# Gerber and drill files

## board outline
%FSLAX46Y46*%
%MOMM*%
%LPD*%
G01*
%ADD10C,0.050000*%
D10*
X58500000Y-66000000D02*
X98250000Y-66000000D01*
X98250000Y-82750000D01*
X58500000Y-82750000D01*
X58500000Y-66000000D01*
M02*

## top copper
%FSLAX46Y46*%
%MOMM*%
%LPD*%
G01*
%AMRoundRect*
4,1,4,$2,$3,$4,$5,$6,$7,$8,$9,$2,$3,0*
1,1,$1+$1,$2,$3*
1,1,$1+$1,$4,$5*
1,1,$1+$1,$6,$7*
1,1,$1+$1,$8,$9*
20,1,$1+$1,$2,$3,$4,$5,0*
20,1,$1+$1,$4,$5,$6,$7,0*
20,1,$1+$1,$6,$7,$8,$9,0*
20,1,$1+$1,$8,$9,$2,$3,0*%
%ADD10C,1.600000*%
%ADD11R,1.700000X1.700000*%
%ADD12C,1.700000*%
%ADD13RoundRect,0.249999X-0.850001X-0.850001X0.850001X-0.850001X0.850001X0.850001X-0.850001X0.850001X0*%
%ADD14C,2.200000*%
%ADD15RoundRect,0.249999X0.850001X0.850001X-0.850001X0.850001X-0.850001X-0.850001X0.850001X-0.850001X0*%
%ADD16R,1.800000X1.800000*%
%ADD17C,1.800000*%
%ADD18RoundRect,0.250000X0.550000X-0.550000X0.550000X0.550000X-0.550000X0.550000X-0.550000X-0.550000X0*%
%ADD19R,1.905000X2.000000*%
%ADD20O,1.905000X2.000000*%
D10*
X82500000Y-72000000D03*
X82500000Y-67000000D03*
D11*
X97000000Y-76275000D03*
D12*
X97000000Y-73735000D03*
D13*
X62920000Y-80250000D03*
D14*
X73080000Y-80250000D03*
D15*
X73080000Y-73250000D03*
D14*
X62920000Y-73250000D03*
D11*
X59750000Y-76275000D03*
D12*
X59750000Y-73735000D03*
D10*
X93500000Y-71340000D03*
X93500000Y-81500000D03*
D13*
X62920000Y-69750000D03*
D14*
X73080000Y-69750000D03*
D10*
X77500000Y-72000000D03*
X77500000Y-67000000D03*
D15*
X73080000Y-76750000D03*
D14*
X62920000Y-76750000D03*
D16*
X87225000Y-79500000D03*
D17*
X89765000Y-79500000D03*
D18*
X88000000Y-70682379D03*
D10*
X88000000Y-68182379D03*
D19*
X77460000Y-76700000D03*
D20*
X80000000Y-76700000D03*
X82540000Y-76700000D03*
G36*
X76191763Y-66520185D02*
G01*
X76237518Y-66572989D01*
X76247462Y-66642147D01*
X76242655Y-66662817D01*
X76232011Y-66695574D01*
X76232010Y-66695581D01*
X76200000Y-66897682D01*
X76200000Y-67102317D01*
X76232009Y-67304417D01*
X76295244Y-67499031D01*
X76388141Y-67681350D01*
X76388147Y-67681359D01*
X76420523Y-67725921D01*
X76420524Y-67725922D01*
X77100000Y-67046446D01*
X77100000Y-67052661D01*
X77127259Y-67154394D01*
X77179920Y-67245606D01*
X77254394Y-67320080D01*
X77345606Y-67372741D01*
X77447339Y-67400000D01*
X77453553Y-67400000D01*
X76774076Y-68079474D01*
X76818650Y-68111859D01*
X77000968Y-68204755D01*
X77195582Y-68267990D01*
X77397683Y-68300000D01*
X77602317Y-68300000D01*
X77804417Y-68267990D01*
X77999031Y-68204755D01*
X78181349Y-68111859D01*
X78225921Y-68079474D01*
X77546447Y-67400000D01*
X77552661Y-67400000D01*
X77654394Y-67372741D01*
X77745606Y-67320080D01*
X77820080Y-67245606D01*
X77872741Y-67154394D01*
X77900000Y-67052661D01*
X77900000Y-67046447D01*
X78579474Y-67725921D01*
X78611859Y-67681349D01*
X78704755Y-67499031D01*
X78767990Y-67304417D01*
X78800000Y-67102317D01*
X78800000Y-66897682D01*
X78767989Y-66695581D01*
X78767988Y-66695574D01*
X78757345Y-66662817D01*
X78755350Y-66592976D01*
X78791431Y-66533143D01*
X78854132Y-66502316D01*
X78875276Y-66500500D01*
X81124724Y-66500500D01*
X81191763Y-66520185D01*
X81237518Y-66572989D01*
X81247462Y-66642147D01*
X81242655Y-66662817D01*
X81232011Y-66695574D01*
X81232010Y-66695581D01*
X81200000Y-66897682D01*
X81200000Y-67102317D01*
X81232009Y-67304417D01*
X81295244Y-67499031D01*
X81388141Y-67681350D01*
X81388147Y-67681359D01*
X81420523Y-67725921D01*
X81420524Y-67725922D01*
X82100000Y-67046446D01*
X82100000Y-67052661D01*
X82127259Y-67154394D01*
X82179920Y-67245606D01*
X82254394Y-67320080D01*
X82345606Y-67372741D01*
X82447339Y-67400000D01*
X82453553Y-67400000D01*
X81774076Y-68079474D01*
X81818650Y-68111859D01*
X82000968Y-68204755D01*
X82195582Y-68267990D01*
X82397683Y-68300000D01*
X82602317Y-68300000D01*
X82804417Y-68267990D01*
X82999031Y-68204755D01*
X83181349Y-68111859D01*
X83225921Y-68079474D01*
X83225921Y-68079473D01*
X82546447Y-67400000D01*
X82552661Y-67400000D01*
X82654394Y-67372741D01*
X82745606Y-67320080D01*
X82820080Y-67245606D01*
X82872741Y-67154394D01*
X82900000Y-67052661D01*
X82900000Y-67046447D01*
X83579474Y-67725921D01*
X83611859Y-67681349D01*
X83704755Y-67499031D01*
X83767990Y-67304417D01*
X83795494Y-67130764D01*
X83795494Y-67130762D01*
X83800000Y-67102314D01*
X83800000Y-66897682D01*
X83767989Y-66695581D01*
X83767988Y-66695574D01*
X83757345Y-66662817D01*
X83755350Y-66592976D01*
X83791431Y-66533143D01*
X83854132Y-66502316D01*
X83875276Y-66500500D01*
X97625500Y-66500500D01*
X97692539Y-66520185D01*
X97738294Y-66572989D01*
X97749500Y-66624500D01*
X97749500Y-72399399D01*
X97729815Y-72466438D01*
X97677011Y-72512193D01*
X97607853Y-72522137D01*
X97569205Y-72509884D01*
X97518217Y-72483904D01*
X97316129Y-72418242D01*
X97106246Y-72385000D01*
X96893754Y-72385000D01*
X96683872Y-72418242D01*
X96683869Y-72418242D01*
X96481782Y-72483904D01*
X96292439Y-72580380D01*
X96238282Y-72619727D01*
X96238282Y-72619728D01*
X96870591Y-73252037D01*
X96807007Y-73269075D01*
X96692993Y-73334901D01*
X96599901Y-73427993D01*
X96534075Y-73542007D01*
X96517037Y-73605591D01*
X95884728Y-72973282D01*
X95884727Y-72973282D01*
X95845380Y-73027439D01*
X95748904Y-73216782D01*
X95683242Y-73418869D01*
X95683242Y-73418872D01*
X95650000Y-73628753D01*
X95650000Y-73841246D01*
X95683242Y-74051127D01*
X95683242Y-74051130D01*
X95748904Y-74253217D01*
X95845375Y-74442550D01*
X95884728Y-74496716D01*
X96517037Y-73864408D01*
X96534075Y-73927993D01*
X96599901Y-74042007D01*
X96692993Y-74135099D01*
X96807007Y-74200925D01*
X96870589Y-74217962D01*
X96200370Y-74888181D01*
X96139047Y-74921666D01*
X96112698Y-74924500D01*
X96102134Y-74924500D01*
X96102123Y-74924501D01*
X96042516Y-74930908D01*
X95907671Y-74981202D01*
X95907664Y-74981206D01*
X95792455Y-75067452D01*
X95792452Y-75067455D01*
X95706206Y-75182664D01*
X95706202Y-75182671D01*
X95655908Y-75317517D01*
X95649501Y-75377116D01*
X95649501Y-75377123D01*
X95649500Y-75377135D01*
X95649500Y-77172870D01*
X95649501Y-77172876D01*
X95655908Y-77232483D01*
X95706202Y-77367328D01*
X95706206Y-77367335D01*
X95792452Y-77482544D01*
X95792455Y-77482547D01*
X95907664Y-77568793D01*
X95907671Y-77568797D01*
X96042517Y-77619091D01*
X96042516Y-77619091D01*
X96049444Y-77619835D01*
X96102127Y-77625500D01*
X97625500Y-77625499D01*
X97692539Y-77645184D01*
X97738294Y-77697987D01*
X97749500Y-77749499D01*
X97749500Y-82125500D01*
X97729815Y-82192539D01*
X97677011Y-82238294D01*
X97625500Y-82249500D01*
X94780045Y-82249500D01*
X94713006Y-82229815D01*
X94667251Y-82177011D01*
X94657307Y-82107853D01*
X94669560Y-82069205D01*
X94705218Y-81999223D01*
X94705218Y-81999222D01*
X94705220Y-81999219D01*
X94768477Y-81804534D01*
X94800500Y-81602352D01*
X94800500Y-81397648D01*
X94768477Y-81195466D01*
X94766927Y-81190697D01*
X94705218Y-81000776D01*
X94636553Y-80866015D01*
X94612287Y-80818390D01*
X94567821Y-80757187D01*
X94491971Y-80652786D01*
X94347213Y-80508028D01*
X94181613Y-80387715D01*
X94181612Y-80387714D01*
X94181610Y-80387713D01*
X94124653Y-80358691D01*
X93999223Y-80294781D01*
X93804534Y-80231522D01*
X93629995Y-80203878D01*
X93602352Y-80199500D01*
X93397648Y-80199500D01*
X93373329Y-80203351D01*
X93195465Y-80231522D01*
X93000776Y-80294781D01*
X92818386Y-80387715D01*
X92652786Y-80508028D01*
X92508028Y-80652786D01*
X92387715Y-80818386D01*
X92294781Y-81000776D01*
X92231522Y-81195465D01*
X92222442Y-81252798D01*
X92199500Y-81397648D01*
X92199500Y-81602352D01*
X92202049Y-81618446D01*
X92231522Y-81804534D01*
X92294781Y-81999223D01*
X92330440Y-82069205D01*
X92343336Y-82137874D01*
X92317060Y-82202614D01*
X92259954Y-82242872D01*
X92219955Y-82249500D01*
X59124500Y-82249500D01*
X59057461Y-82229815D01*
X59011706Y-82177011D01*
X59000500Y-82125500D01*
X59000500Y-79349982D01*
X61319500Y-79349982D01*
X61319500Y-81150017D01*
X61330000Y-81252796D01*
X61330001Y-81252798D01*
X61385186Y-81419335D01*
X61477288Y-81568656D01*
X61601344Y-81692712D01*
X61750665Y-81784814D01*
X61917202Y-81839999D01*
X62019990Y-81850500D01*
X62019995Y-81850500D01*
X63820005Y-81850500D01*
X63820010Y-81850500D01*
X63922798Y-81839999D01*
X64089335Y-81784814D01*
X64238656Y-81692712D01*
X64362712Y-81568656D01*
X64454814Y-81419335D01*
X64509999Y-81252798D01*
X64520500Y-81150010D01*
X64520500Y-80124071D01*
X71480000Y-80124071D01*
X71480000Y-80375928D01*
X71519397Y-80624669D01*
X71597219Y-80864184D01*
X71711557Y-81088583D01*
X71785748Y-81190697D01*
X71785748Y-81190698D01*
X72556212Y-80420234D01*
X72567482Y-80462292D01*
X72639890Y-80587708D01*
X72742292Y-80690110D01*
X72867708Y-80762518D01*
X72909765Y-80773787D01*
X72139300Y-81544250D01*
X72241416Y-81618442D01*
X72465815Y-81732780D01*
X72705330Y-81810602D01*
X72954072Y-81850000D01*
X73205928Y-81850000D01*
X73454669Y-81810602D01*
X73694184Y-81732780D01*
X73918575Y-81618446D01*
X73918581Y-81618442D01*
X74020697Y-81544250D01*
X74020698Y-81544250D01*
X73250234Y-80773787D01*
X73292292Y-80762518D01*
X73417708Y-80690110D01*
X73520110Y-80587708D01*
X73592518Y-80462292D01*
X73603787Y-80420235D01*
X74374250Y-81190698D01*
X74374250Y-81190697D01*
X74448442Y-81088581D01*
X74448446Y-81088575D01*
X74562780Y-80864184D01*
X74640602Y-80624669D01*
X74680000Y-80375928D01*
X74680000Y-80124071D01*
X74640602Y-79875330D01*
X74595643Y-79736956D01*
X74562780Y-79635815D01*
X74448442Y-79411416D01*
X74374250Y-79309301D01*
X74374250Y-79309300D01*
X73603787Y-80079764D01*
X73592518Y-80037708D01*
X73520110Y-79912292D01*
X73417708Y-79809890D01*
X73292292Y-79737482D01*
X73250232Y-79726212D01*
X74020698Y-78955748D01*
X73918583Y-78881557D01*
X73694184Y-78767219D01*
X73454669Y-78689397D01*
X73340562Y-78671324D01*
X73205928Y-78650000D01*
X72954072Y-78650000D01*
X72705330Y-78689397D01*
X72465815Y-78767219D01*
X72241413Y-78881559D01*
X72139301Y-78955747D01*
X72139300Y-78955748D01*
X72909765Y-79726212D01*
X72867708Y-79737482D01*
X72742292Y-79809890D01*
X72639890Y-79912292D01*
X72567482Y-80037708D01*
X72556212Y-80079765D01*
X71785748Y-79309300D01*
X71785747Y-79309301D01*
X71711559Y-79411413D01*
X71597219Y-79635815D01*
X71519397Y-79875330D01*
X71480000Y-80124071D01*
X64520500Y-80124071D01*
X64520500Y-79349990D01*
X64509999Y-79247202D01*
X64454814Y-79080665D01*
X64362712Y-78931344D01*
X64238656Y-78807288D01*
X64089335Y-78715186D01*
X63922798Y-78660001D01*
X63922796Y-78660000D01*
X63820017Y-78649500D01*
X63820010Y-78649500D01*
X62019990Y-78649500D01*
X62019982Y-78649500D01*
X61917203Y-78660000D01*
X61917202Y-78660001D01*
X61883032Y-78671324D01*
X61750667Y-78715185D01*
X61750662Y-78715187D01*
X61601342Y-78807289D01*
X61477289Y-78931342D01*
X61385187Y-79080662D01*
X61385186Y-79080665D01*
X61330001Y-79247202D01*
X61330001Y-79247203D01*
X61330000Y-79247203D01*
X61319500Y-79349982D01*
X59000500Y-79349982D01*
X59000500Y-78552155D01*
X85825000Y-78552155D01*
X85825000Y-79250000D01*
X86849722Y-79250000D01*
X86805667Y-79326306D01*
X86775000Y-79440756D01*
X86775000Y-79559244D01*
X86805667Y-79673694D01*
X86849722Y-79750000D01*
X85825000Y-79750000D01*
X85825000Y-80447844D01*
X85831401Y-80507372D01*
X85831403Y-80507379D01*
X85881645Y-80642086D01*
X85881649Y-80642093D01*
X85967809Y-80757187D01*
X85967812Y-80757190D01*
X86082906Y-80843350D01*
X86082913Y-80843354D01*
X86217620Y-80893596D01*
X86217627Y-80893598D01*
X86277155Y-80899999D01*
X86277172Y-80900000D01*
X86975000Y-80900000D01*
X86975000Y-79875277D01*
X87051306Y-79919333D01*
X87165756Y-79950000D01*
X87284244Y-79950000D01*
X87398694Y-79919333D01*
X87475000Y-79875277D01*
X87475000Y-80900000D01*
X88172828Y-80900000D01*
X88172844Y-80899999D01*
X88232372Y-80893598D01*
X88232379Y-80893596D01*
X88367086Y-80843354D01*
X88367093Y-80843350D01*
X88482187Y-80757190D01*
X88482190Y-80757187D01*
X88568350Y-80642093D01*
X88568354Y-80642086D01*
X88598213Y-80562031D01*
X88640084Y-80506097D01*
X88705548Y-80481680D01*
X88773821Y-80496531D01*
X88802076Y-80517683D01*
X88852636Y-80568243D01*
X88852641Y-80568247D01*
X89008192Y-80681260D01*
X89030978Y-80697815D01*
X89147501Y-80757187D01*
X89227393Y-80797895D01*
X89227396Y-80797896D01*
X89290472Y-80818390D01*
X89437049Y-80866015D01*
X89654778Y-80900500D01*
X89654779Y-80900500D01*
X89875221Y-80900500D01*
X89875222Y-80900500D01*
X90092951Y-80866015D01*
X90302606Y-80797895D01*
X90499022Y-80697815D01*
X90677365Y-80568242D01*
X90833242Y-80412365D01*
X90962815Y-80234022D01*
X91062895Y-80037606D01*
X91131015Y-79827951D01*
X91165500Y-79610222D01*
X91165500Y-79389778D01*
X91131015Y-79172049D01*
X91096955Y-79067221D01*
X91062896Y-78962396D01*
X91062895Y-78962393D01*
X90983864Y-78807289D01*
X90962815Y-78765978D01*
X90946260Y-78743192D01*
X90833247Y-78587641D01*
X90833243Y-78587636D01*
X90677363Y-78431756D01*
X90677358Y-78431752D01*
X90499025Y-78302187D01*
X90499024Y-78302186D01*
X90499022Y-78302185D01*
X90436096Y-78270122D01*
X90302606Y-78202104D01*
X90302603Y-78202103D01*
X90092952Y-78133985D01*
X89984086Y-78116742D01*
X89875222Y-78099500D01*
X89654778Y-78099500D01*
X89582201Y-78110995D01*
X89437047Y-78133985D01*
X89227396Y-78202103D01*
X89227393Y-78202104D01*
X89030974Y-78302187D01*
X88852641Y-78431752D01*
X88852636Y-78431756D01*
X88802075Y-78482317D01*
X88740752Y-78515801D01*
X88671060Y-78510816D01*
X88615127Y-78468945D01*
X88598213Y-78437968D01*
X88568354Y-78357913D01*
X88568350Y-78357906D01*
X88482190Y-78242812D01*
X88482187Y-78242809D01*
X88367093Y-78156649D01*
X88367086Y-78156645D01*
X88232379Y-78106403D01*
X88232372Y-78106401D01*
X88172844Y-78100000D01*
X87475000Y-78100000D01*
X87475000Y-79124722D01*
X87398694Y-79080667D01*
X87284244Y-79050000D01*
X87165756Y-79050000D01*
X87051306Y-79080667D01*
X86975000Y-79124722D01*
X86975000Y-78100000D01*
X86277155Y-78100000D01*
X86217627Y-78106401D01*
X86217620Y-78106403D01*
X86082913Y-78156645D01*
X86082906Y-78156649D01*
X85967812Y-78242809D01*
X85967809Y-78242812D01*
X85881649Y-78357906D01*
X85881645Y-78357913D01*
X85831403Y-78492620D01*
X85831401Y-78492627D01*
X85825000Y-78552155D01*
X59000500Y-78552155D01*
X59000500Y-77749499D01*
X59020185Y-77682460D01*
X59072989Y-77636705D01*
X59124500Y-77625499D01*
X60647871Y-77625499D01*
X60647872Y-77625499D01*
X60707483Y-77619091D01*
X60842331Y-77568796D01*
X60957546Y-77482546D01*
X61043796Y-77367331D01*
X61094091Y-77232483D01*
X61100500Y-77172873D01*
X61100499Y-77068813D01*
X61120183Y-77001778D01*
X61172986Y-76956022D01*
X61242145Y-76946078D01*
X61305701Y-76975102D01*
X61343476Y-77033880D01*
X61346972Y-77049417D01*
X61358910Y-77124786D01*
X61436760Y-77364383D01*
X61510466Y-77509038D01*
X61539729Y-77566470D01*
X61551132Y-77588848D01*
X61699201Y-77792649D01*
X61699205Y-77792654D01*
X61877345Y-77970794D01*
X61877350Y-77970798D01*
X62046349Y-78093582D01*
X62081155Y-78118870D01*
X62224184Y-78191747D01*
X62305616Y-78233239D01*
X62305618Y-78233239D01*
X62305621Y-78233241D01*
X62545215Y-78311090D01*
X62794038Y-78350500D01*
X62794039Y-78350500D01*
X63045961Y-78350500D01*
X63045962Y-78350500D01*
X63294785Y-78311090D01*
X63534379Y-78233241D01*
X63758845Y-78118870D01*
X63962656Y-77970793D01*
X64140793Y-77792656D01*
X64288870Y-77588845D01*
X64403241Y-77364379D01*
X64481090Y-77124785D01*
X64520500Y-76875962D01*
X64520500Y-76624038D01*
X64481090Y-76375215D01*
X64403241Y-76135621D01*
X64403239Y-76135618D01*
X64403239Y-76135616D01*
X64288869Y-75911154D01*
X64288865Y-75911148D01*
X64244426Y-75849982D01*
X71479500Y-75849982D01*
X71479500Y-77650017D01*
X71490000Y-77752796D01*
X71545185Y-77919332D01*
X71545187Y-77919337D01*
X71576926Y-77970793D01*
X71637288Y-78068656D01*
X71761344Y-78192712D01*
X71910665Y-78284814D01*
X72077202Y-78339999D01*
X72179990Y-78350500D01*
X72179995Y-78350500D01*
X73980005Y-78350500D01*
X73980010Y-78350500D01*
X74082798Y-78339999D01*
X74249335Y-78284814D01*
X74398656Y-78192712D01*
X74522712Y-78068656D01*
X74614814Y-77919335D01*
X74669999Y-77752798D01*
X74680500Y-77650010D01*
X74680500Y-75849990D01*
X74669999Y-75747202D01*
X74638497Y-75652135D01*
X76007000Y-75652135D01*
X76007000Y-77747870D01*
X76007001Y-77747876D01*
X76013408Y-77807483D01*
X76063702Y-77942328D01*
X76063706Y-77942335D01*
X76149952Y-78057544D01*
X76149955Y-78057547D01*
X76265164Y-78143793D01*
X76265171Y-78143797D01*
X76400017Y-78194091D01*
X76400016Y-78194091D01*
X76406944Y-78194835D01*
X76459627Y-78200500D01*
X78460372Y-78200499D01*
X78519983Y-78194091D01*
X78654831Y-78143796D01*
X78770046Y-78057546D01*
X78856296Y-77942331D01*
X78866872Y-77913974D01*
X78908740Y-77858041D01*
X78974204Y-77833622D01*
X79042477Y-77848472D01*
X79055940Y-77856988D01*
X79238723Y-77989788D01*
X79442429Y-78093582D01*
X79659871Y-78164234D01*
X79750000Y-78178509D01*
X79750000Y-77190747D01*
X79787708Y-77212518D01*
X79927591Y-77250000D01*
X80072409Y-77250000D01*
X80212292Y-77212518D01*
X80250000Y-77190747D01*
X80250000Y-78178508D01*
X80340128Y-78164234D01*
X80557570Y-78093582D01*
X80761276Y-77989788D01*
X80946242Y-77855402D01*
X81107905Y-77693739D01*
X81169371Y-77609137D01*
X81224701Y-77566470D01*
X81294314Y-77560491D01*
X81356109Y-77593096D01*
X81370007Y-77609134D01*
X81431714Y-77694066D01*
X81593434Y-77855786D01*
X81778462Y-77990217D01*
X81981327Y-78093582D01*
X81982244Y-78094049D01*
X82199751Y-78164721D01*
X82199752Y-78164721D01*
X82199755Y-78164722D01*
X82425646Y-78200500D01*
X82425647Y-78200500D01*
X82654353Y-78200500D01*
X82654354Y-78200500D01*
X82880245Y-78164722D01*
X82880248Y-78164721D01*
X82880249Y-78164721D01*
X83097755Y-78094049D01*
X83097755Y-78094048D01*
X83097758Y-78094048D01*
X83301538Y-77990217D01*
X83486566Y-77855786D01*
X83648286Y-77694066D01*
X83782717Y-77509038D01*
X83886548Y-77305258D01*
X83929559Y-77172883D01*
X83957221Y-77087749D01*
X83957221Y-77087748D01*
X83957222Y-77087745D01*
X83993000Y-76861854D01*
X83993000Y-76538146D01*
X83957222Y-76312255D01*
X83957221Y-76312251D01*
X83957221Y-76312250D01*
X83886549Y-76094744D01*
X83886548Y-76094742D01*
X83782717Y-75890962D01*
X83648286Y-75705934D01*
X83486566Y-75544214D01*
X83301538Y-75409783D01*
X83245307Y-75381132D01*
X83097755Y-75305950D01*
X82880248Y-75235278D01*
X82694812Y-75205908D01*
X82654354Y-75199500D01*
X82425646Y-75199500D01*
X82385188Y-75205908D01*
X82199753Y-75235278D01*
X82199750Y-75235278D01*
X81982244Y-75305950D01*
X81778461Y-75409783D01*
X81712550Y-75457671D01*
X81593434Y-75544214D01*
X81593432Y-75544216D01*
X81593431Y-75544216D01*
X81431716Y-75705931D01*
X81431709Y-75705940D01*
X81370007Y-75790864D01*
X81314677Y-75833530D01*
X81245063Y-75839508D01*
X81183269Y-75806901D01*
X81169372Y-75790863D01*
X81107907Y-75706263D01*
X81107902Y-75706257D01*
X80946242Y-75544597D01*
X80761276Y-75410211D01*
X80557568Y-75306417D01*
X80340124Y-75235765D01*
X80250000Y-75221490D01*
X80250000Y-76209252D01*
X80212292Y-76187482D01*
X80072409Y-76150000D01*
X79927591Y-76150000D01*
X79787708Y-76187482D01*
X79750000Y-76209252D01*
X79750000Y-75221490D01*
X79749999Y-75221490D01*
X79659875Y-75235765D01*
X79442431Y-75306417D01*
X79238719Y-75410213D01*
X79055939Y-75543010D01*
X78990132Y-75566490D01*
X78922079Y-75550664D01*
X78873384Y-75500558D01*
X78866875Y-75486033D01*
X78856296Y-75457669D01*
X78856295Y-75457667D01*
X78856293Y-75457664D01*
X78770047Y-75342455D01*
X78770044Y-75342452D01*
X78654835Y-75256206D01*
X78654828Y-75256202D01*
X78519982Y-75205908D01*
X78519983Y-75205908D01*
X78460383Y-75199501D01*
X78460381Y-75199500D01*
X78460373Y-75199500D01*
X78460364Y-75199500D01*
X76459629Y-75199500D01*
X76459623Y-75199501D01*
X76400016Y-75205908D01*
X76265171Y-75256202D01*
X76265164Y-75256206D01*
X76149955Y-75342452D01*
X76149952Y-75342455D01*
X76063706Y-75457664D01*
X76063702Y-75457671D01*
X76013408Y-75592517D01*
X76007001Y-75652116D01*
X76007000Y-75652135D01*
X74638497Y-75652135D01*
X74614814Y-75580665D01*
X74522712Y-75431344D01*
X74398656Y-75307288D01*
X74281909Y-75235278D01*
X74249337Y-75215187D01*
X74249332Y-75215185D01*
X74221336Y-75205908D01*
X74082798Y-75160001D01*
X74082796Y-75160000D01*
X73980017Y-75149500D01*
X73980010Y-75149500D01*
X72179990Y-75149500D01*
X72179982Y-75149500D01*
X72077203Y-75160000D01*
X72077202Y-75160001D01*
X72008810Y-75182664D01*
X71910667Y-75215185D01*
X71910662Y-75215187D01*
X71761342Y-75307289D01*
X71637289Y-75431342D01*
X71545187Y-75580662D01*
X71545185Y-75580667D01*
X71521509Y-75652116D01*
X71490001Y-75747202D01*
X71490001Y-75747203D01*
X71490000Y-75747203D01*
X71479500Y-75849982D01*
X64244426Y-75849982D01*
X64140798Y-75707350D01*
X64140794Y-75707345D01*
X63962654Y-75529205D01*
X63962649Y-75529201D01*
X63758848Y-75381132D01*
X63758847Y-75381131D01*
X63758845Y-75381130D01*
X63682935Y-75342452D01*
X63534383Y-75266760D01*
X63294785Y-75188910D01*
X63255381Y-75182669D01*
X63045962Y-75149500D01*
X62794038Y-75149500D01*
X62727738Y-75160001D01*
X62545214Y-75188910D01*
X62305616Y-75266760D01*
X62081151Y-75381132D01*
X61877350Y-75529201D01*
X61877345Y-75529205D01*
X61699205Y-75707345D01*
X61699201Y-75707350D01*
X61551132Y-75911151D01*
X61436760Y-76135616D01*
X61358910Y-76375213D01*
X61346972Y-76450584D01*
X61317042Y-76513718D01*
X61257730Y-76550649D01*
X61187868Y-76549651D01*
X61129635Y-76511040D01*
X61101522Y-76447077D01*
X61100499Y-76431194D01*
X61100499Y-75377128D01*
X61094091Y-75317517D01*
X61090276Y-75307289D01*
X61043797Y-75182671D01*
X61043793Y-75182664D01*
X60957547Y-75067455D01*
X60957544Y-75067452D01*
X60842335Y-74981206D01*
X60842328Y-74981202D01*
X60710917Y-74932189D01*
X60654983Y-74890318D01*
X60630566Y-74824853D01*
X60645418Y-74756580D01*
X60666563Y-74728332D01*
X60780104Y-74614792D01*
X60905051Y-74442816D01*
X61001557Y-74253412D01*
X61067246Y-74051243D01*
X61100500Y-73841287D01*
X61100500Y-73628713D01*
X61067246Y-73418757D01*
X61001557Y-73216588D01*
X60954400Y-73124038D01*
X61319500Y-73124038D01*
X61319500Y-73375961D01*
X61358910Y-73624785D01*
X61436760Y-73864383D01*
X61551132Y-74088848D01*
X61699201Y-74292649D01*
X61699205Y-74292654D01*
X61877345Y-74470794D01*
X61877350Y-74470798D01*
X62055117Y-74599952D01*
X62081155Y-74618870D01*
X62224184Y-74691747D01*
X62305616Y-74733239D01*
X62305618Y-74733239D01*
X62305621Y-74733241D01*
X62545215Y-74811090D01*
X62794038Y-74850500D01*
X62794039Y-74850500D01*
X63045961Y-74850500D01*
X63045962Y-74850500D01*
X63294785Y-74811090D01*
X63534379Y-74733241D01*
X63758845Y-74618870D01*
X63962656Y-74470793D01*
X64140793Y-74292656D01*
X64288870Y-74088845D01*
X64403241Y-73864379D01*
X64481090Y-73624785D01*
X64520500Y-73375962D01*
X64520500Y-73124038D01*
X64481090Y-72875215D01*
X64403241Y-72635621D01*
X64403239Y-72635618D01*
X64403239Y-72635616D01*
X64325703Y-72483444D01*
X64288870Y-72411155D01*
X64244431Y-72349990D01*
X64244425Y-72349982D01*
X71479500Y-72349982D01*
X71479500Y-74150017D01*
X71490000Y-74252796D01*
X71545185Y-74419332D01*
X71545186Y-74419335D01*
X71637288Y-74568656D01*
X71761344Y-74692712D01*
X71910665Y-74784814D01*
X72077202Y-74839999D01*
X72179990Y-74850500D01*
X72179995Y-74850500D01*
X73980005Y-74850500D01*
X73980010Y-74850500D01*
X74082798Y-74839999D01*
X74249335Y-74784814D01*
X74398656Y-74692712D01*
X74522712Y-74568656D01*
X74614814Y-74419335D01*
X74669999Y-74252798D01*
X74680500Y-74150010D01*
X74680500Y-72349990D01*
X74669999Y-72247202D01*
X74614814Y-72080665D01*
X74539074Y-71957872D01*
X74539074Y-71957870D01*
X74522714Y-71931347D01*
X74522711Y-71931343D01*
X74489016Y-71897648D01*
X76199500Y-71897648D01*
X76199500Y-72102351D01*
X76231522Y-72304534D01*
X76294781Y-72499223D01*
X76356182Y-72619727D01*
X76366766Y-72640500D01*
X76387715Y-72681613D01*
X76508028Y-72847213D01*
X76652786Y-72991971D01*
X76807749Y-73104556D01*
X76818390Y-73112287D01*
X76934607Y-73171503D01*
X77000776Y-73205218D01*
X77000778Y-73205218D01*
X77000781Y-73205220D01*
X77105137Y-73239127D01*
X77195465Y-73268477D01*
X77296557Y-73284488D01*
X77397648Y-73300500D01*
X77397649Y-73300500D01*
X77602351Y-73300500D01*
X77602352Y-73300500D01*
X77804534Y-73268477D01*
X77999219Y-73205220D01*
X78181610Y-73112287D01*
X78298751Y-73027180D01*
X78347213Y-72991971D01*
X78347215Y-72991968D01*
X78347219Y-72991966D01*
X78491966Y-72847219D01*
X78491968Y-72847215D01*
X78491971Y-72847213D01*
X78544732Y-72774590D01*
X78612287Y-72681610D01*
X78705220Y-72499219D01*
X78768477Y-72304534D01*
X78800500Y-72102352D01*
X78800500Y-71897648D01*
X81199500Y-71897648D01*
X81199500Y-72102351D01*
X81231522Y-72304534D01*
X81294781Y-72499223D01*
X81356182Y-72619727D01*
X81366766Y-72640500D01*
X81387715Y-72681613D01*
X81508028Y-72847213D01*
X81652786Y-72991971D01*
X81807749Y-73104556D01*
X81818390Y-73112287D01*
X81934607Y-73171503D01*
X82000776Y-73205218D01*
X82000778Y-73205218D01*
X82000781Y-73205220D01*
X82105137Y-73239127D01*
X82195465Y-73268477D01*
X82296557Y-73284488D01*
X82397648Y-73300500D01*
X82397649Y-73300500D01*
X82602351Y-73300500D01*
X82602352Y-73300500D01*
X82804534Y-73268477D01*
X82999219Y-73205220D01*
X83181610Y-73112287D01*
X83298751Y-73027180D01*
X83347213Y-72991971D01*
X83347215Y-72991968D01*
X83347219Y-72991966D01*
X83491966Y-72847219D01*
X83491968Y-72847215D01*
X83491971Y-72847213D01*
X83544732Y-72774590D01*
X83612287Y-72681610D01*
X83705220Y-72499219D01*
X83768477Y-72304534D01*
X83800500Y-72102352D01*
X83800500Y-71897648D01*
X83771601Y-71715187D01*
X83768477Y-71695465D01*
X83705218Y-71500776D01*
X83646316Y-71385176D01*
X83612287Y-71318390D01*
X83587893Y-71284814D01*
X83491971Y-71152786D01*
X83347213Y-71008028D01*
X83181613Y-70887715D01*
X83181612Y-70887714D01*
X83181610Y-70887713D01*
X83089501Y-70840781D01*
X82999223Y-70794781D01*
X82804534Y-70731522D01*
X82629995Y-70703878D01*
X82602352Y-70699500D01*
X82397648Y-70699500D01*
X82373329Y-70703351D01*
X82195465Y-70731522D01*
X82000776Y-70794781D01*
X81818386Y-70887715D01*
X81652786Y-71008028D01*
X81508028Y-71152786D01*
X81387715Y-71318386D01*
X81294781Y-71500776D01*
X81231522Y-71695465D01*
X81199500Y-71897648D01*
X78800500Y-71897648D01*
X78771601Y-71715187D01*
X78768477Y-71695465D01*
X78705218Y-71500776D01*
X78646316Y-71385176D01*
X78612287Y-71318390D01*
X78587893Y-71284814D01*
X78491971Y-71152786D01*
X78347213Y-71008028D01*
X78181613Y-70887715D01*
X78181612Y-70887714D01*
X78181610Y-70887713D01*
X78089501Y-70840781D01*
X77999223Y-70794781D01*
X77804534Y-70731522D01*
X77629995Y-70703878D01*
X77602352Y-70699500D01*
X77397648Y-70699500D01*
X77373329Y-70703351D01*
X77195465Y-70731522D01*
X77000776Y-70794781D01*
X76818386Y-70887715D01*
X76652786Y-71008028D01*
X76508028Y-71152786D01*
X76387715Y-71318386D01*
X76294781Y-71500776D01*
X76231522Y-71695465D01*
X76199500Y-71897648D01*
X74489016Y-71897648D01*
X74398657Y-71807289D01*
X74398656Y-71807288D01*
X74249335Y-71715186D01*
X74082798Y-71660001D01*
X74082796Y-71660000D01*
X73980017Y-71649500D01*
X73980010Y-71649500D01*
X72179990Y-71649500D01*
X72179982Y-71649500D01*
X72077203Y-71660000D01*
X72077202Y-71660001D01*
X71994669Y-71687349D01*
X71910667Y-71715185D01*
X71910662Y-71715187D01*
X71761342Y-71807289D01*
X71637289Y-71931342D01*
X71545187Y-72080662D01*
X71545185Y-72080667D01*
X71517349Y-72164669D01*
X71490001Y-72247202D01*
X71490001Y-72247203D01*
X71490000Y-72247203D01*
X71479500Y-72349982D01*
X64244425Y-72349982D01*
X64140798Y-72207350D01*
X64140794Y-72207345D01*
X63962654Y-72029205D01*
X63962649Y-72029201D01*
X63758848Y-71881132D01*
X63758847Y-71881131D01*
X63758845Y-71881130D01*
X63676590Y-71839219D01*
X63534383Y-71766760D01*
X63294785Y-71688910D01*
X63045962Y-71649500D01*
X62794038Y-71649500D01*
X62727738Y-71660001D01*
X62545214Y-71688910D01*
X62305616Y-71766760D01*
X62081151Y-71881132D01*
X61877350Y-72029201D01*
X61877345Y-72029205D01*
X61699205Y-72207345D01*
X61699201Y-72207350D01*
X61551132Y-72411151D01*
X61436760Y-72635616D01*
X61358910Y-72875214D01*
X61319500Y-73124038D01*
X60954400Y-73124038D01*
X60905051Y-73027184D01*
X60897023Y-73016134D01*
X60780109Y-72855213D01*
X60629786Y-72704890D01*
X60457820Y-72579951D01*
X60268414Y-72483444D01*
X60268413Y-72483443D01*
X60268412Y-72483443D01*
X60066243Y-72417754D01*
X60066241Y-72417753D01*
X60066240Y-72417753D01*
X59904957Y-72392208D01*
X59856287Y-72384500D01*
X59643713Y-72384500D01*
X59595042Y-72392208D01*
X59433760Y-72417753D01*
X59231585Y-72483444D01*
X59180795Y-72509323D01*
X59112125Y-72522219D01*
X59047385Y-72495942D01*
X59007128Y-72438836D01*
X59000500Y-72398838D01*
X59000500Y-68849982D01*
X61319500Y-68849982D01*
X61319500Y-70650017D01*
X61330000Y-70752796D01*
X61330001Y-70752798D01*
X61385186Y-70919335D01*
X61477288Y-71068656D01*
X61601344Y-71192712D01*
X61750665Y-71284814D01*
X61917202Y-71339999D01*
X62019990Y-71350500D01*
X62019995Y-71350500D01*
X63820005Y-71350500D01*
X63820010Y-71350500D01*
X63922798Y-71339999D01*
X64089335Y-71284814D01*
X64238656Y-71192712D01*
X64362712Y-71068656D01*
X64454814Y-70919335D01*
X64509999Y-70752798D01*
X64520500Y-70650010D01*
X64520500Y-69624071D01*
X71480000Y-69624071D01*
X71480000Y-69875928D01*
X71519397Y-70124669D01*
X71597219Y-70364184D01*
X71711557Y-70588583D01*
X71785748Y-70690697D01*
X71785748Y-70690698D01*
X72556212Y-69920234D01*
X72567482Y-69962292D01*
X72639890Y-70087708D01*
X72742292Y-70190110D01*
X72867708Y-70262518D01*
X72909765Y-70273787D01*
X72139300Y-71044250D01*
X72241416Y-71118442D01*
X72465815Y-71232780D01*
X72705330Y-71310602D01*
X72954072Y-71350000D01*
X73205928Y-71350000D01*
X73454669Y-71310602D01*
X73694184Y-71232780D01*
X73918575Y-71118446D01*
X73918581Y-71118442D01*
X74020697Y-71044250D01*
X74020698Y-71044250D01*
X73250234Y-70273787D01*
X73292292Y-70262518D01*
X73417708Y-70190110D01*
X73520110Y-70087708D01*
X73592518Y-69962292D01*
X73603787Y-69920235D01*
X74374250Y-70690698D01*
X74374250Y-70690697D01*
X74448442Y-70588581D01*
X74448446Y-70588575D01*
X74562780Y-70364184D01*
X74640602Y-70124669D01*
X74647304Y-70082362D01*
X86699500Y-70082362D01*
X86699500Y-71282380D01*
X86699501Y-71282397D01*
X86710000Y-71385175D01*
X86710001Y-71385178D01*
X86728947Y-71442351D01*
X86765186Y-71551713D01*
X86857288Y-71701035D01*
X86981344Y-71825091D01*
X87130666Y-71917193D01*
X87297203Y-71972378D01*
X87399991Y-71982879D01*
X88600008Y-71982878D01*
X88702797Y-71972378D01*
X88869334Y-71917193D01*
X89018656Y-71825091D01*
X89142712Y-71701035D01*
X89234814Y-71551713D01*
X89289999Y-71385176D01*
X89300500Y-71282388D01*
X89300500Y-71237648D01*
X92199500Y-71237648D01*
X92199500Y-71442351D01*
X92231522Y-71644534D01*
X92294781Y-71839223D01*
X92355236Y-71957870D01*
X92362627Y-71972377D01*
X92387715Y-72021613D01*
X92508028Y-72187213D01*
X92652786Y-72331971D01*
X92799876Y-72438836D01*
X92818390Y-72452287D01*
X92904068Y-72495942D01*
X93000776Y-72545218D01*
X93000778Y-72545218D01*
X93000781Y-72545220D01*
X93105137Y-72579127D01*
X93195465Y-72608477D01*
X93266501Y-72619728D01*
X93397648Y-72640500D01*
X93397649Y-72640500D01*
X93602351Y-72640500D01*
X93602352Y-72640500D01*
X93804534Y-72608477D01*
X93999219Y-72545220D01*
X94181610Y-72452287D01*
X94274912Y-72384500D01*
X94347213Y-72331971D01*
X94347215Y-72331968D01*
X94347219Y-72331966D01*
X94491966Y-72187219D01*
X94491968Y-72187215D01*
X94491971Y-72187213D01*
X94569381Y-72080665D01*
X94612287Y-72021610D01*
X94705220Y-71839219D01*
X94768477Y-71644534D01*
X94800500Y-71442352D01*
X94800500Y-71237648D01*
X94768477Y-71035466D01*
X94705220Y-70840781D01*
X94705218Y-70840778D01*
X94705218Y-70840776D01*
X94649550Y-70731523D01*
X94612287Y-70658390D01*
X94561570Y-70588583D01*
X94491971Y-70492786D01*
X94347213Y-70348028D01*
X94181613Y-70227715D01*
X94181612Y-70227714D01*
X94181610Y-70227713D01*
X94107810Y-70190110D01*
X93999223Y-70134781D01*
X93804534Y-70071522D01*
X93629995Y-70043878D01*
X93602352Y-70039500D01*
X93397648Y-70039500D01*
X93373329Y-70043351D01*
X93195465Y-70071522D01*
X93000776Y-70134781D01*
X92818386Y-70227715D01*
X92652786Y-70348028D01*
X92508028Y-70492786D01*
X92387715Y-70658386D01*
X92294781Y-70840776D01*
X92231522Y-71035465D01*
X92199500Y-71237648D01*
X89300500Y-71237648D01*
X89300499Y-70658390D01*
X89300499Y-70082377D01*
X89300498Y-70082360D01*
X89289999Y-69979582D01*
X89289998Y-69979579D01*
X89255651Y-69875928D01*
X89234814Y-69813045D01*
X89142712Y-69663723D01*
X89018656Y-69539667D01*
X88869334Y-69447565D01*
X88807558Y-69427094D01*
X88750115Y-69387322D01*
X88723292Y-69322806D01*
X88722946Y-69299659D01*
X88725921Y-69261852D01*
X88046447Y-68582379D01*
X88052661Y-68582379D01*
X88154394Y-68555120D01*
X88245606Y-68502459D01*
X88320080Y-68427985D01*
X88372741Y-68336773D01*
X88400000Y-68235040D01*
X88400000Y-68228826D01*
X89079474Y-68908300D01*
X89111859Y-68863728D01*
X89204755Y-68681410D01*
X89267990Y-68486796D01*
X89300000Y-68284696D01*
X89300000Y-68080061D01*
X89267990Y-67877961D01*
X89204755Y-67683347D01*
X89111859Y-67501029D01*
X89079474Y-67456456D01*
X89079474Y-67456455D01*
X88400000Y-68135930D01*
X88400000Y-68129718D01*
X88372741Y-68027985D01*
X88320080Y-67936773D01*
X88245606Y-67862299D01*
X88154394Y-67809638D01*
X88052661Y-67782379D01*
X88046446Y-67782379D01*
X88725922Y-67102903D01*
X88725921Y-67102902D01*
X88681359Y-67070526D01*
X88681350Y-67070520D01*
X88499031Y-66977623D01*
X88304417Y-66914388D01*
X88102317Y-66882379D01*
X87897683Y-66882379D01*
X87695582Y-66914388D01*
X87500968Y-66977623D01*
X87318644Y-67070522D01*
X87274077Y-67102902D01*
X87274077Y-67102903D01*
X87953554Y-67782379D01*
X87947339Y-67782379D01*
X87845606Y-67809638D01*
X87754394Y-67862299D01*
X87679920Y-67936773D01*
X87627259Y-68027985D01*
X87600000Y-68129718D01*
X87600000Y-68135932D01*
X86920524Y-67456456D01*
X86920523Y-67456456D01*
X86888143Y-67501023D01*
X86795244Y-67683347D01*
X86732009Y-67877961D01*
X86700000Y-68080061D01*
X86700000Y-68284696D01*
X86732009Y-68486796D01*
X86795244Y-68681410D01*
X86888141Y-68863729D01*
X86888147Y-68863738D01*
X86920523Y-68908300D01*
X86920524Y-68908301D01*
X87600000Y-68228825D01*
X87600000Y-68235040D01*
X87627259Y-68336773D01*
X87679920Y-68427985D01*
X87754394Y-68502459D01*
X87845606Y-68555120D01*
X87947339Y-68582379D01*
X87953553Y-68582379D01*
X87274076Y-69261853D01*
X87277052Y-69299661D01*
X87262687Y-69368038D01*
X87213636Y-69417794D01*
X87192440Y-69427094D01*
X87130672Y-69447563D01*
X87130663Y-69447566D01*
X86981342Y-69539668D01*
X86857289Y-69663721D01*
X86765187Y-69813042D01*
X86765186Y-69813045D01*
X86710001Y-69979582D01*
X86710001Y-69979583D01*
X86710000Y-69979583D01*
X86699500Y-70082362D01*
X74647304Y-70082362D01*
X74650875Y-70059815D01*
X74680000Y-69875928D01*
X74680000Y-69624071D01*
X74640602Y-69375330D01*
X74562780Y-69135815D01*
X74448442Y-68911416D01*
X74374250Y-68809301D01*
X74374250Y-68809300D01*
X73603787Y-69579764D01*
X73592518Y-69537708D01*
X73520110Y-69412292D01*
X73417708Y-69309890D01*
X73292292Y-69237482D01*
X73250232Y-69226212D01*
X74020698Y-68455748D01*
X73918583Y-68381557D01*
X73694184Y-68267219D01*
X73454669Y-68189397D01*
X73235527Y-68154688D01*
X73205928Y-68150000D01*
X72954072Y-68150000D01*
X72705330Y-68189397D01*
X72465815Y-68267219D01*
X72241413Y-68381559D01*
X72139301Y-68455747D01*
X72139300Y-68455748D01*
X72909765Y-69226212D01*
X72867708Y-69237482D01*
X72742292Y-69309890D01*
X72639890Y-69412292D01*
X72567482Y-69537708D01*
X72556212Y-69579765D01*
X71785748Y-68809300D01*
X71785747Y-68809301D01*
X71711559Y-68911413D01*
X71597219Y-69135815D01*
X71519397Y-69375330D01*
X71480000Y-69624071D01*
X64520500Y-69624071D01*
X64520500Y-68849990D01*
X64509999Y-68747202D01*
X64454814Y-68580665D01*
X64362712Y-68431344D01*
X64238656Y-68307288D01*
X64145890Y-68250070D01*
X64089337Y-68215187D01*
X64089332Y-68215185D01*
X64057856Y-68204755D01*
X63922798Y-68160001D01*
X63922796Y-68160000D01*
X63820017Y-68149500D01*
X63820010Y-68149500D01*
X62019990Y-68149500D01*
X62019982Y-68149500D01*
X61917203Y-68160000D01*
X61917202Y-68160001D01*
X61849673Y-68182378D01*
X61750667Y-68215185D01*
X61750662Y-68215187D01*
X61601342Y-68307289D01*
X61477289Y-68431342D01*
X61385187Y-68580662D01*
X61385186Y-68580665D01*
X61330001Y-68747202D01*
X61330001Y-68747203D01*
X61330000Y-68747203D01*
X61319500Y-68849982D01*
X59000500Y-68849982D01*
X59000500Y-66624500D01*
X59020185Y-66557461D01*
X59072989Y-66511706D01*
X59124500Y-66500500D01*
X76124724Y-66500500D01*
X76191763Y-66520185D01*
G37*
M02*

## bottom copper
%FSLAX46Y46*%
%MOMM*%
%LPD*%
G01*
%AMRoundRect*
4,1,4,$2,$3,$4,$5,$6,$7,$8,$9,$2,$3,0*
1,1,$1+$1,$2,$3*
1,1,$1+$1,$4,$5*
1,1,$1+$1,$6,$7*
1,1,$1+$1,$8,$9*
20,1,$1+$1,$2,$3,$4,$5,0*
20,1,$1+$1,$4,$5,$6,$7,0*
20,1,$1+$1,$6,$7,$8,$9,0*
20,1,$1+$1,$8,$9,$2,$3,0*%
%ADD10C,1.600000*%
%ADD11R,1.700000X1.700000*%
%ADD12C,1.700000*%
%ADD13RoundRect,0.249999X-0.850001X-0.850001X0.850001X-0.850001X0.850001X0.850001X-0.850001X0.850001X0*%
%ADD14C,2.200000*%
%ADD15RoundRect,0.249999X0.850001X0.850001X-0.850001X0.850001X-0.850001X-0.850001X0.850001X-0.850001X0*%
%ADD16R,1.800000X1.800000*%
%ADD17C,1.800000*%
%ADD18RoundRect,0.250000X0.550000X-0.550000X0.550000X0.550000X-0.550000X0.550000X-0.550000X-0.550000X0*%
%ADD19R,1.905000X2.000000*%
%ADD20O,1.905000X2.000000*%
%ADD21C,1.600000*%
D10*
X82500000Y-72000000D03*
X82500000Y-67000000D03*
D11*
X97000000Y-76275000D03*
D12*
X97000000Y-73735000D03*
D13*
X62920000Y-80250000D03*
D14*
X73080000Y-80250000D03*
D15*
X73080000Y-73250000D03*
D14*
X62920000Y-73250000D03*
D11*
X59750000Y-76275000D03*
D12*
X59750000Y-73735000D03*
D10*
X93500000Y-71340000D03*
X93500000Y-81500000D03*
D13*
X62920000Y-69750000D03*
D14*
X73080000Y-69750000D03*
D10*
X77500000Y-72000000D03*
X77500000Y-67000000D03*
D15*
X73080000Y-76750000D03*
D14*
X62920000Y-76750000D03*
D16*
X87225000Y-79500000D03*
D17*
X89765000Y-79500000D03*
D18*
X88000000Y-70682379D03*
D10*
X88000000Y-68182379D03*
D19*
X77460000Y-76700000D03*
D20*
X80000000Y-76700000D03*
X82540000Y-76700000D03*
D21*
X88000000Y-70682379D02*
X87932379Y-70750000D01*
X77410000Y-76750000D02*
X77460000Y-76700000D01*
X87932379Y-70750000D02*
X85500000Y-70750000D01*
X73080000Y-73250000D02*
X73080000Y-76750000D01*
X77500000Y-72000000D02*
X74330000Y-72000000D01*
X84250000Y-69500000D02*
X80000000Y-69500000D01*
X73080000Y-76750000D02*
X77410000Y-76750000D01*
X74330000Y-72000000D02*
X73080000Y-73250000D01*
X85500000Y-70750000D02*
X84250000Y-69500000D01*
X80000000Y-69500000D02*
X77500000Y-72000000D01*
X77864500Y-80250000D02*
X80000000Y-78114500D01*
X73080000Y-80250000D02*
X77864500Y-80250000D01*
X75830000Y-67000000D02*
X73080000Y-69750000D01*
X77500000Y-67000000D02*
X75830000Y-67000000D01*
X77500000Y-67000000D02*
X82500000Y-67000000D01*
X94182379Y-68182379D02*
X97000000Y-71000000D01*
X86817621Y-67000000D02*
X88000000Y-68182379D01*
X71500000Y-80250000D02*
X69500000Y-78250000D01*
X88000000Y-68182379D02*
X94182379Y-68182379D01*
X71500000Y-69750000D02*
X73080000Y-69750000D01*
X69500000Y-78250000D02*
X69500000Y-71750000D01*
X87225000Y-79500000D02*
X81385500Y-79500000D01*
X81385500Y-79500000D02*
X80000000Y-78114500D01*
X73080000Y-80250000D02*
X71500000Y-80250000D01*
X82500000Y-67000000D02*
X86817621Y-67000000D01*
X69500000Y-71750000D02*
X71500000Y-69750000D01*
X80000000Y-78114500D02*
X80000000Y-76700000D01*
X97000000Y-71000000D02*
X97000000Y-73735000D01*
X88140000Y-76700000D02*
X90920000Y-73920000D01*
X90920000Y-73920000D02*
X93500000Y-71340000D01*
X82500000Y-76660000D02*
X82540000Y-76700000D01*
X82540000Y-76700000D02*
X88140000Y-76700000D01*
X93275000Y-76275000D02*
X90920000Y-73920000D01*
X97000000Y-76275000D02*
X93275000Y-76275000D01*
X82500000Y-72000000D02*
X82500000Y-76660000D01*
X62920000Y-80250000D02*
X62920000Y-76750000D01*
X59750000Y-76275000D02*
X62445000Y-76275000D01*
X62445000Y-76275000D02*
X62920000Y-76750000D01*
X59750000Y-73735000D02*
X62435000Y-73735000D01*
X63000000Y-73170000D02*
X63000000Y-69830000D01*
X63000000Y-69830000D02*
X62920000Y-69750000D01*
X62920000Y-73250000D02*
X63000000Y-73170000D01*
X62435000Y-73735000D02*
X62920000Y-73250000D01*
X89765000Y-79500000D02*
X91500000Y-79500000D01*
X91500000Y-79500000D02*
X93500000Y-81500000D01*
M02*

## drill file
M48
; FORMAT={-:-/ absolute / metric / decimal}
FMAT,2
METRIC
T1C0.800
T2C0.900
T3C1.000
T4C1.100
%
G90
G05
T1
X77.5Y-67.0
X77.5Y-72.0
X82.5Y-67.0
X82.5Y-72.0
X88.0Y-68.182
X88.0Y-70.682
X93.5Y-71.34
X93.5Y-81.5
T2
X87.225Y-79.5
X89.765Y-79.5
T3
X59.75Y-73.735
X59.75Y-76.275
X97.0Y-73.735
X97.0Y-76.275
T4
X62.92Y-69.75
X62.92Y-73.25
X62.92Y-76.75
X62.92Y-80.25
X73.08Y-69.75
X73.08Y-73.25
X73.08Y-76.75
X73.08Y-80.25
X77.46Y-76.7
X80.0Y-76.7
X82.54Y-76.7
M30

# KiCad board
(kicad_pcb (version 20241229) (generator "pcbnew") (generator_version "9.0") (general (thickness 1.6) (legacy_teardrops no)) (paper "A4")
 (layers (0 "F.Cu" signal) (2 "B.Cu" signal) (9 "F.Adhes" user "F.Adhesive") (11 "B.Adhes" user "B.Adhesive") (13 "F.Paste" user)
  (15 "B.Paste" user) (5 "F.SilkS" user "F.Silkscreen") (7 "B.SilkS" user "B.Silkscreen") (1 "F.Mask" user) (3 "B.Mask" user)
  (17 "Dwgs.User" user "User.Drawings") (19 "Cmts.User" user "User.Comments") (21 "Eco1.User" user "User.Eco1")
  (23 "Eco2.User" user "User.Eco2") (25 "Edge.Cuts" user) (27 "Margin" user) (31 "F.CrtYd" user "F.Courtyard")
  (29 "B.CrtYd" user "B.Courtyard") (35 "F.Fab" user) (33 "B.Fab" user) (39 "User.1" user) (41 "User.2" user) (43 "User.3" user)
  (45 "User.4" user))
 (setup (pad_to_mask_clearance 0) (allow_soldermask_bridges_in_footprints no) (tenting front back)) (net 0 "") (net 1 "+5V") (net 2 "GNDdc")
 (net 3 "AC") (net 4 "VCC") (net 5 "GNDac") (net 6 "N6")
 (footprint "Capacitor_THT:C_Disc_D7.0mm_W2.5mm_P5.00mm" (layer "F.Cu") (at 82.5 72 90)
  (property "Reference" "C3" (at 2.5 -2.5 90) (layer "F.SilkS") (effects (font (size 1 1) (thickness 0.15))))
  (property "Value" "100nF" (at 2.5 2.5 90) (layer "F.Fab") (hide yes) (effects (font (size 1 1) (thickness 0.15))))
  (pad "1" thru_hole circle (at 0 0 90) (size 1.6 1.6) (drill 0.8) (layers "*.Cu" "*.Mask") (remove_unused_layers no) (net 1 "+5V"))
  (pad "2" thru_hole circle (at 5 0 90) (size 1.6 1.6) (drill 0.8) (layers "*.Cu" "*.Mask") (remove_unused_layers no) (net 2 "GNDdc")))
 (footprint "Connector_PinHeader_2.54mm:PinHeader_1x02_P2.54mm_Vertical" (layer "F.Cu") (at 97 76.275 180)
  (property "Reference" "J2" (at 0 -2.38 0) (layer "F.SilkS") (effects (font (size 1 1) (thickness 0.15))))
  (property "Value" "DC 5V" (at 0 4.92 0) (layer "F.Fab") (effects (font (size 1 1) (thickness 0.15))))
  (pad "1" thru_hole rect (at 0 0 180) (size 1.7 1.7) (drill 1) (layers "*.Cu" "*.Mask") (remove_unused_layers no) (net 1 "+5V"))
  (pad "2" thru_hole circle (at 0 2.54 180) (size 1.7 1.7) (drill 1) (layers "*.Cu" "*.Mask") (remove_unused_layers no) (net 2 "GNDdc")))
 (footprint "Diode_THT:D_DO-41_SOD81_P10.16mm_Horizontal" (layer "F.Cu") (at 62.92 80.25)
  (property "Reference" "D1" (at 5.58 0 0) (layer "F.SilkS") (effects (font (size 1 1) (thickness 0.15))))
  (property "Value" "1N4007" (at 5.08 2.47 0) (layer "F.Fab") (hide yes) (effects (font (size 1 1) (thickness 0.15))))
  (pad "1" thru_hole roundrect (at 0 0) (size 2.2 2.2) (drill 1.1) (layers "*.Cu" "*.Mask") (remove_unused_layers no)
   (roundrect_rratio 0.113636) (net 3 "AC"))
  (pad "2" thru_hole circle (at 10.16 0) (size 2.2 2.2) (drill 1.1) (layers "*.Cu" "*.Mask") (remove_unused_layers no) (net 2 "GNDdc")))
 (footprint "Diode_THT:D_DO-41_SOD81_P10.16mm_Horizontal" (layer "F.Cu") (at 73.08 73.25 180)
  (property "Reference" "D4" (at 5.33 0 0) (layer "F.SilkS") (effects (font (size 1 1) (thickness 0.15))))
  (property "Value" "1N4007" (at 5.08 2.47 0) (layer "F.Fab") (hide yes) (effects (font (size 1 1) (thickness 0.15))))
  (pad "1" thru_hole roundrect (at 0 0 180) (size 2.2 2.2) (drill 1.1) (layers "*.Cu" "*.Mask") (remove_unused_layers no)
   (roundrect_rratio 0.113636) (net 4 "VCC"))
  (pad "2" thru_hole circle (at 10.16 0 180) (size 2.2 2.2) (drill 1.1) (layers "*.Cu" "*.Mask") (remove_unused_layers no) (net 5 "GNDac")))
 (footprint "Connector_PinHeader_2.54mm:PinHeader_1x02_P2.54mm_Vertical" (layer "F.Cu") (at 59.75 76.275 180)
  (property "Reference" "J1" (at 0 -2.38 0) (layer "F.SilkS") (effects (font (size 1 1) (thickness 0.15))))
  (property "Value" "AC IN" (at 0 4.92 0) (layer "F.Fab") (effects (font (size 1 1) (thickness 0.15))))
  (pad "1" thru_hole rect (at 0 0 180) (size 1.7 1.7) (drill 1) (layers "*.Cu" "*.Mask") (remove_unused_layers no) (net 3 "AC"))
  (pad "2" thru_hole circle (at 0 2.54 180) (size 1.7 1.7) (drill 1) (layers "*.Cu" "*.Mask") (remove_unused_layers no) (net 5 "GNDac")))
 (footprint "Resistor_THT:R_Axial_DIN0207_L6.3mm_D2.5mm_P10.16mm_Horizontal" (layer "F.Cu") (at 93.5 71.34 -90)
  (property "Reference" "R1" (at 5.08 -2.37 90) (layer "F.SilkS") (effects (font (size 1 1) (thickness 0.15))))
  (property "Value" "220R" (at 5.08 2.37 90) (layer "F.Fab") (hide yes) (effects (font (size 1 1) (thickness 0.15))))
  (pad "1" thru_hole circle (at 0 0 270) (size 1.6 1.6) (drill 0.8) (layers "*.Cu" "*.Mask") (remove_unused_layers no) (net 1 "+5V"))
  (pad "2" thru_hole circle (at 10.16 0 270) (size 1.6 1.6) (drill 0.8) (layers "*.Cu" "*.Mask") (remove_unused_layers no) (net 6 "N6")))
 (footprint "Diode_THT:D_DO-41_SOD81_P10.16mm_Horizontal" (layer "F.Cu") (at 62.92 69.75)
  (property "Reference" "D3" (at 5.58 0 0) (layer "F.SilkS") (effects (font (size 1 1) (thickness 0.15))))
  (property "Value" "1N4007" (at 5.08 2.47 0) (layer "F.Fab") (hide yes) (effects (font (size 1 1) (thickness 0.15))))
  (pad "1" thru_hole roundrect (at 0 0) (size 2.2 2.2) (drill 1.1) (layers "*.Cu" "*.Mask") (remove_unused_layers no)
   (roundrect_rratio 0.113636) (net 5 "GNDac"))
  (pad "2" thru_hole circle (at 10.16 0) (size 2.2 2.2) (drill 1.1) (layers "*.Cu" "*.Mask") (remove_unused_layers no) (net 2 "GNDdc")))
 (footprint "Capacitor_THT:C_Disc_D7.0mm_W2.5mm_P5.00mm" (layer "F.Cu") (at 77.5 72 90)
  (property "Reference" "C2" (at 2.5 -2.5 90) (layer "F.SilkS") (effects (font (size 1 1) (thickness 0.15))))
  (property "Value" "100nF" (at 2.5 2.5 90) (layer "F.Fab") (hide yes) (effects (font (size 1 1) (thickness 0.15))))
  (pad "1" thru_hole circle (at 0 0 90) (size 1.6 1.6) (drill 0.8) (layers "*.Cu" "*.Mask") (remove_unused_layers no) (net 4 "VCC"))
  (pad "2" thru_hole circle (at 5 0 90) (size 1.6 1.6) (drill 0.8) (layers "*.Cu" "*.Mask") (remove_unused_layers no) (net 2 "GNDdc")))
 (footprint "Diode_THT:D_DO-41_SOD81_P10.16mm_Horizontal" (layer "F.Cu") (at 73.08 76.75 180)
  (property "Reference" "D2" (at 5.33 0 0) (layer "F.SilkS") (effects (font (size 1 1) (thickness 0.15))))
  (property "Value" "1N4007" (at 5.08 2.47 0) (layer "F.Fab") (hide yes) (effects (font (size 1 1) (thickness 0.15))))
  (pad "1" thru_hole roundrect (at 0 0 180) (size 2.2 2.2) (drill 1.1) (layers "*.Cu" "*.Mask") (remove_unused_layers no)
   (roundrect_rratio 0.113636) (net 4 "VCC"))
  (pad "2" thru_hole circle (at 10.16 0 180) (size 2.2 2.2) (drill 1.1) (layers "*.Cu" "*.Mask") (remove_unused_layers no) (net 3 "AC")))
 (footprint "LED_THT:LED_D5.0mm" (layer "F.Cu") (at 87.225 79.5)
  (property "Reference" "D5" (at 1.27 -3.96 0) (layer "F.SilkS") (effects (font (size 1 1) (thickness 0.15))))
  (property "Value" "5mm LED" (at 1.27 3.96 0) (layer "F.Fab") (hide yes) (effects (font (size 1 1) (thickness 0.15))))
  (pad "1" thru_hole rect (at 0 0) (size 1.8 1.8) (drill 0.9) (layers "*.Cu" "*.Mask") (remove_unused_layers no) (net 2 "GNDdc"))
  (pad "2" thru_hole circle (at 2.54 0) (size 1.8 1.8) (drill 0.9) (layers "*.Cu" "*.Mask") (remove_unused_layers no) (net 6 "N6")))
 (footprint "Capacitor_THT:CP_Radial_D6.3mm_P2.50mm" (layer "F.Cu") (at 88 70.682379 90)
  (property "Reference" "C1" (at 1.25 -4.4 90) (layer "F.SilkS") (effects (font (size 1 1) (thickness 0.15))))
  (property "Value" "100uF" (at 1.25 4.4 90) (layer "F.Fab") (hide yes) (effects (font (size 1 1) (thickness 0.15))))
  (pad "1" thru_hole roundrect (at 0 0 90) (size 1.6 1.6) (drill 0.8) (layers "*.Cu" "*.Mask") (remove_unused_layers no)
   (roundrect_rratio 0.15625) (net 4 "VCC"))
  (pad "2" thru_hole circle (at 2.5 0 90) (size 1.6 1.6) (drill 0.8) (layers "*.Cu" "*.Mask") (remove_unused_layers no) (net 2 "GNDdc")))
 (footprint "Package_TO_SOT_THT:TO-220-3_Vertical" (layer "F.Cu") (at 77.46 76.7)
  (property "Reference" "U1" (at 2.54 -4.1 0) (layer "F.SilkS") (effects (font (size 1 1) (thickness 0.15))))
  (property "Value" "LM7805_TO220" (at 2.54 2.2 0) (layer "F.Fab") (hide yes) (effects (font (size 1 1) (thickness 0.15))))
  (pad "1" thru_hole rect (at 0 0) (size 1.905 2) (drill 1.1) (layers "*.Cu" "*.Mask") (remove_unused_layers no) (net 4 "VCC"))
  (pad "2" thru_hole oval (at 2.54 0) (size 1.905 2) (drill 1.1) (layers "*.Cu" "*.Mask") (remove_unused_layers no) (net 2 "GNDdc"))
  (pad "3" thru_hole oval (at 5.08 0) (size 1.905 2) (drill 1.1) (layers "*.Cu" "*.Mask") (remove_unused_layers no) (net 1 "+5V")))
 (gr_rect (start 58.5 66) (end 98.25 82.75) (stroke (width 0.05) (type default)) (fill no) (layer "Edge.Cuts"))
 (segment (start 88 70.682379) (end 87.932379 70.75) (width 1.6) (layer "B.Cu") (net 4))
 (segment (start 77.41 76.75) (end 77.46 76.7) (width 1.6) (layer "B.Cu") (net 4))
 (segment (start 87.932379 70.75) (end 85.5 70.75) (width 1.6) (layer "B.Cu") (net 4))
 (segment (start 73.08 73.25) (end 73.08 76.75) (width 1.6) (layer "B.Cu") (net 4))
 (segment (start 77.5 72) (end 74.33 72) (width 1.6) (layer "B.Cu") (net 4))
 (segment (start 84.25 69.5) (end 80 69.5) (width 1.6) (layer "B.Cu") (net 4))
 (segment (start 73.08 76.75) (end 77.41 76.75) (width 1.6) (layer "B.Cu") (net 4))
 (segment (start 74.33 72) (end 73.08 73.25) (width 1.6) (layer "B.Cu") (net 4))
 (segment (start 85.5 70.75) (end 84.25 69.5) (width 1.6) (layer "B.Cu") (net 4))
 (segment (start 80 69.5) (end 77.5 72) (width 1.6) (layer "B.Cu") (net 4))
 (segment (start 77.8645 80.25) (end 80 78.1145) (width 1.6) (layer "B.Cu") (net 2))
 (segment (start 73.08 80.25) (end 77.8645 80.25) (width 1.6) (layer "B.Cu") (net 2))
 (segment (start 75.83 67) (end 73.08 69.75) (width 1.6) (layer "B.Cu") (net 2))
 (segment (start 77.5 67) (end 75.83 67) (width 1.6) (layer "B.Cu") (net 2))
 (segment (start 77.5 67) (end 82.5 67) (width 1.6) (layer "B.Cu") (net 2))
 (segment (start 94.182379 68.182379) (end 97 71) (width 1.6) (layer "B.Cu") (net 2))
 (segment (start 86.817621 67) (end 88 68.182379) (width 1.6) (layer "B.Cu") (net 2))
 (segment (start 71.5 80.25) (end 69.5 78.25) (width 1.6) (layer "B.Cu") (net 2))
 (segment (start 88 68.182379) (end 94.182379 68.182379) (width 1.6) (layer "B.Cu") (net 2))
 (segment (start 71.5 69.75) (end 73.08 69.75) (width 1.6) (layer "B.Cu") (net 2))
 (segment (start 69.5 78.25) (end 69.5 71.75) (width 1.6) (layer "B.Cu") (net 2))
 (segment (start 87.225 79.5) (end 81.3855 79.5) (width 1.6) (layer "B.Cu") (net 2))
 (segment (start 81.3855 79.5) (end 80 78.1145) (width 1.6) (layer "B.Cu") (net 2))
 (segment (start 73.08 80.25) (end 71.5 80.25) (width 1.6) (layer "B.Cu") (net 2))
 (segment (start 82.5 67) (end 86.817621 67) (width 1.6) (layer "B.Cu") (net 2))
 (segment (start 69.5 71.75) (end 71.5 69.75) (width 1.6) (layer "B.Cu") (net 2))
 (segment (start 80 78.1145) (end 80 76.7) (width 1.6) (layer "B.Cu") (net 2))
 (segment (start 97 71) (end 97 73.735) (width 1.6) (layer "B.Cu") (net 2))
 (segment (start 88.14 76.7) (end 90.92 73.92) (width 1.6) (layer "B.Cu") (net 1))
 (segment (start 90.92 73.92) (end 93.5 71.34) (width 1.6) (layer "B.Cu") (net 1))
 (segment (start 82.5 76.66) (end 82.54 76.7) (width 1.6) (layer "B.Cu") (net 1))
 (segment (start 82.54 76.7) (end 88.14 76.7) (width 1.6) (layer "B.Cu") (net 1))
 (segment (start 93.275 76.275) (end 90.92 73.92) (width 1.6) (layer "B.Cu") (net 1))
 (segment (start 97 76.275) (end 93.275 76.275) (width 1.6) (layer "B.Cu") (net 1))
 (segment (start 82.5 72) (end 82.5 76.66) (width 1.6) (layer "B.Cu") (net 1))
 (segment (start 62.92 80.25) (end 62.92 76.75) (width 1.6) (layer "B.Cu") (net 3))
 (segment (start 59.75 76.275) (end 62.445 76.275) (width 1.6) (layer "B.Cu") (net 3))
 (segment (start 62.445 76.275) (end 62.92 76.75) (width 1.6) (layer "B.Cu") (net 3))
 (segment (start 59.75 73.735) (end 62.435 73.735) (width 1.6) (layer "B.Cu") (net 5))
 (segment (start 63 73.17) (end 63 69.83) (width 1.6) (layer "B.Cu") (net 5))
 (segment (start 63 69.83) (end 62.92 69.75) (width 1.6) (layer "B.Cu") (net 5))
 (segment (start 62.92 73.25) (end 63 73.17) (width 1.6) (layer "B.Cu") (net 5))
 (segment (start 62.435 73.735) (end 62.92 73.25) (width 1.6) (layer "B.Cu") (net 5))
 (segment (start 89.765 79.5) (end 91.5 79.5) (width 1.6) (layer "B.Cu") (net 6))
 (segment (start 91.5 79.5) (end 93.5 81.5) (width 1.6) (layer "B.Cu") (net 6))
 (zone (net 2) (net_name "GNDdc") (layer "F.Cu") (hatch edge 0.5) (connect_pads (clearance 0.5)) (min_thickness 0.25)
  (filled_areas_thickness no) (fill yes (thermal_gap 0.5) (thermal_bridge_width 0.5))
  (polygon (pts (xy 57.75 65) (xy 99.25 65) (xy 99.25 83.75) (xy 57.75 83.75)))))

